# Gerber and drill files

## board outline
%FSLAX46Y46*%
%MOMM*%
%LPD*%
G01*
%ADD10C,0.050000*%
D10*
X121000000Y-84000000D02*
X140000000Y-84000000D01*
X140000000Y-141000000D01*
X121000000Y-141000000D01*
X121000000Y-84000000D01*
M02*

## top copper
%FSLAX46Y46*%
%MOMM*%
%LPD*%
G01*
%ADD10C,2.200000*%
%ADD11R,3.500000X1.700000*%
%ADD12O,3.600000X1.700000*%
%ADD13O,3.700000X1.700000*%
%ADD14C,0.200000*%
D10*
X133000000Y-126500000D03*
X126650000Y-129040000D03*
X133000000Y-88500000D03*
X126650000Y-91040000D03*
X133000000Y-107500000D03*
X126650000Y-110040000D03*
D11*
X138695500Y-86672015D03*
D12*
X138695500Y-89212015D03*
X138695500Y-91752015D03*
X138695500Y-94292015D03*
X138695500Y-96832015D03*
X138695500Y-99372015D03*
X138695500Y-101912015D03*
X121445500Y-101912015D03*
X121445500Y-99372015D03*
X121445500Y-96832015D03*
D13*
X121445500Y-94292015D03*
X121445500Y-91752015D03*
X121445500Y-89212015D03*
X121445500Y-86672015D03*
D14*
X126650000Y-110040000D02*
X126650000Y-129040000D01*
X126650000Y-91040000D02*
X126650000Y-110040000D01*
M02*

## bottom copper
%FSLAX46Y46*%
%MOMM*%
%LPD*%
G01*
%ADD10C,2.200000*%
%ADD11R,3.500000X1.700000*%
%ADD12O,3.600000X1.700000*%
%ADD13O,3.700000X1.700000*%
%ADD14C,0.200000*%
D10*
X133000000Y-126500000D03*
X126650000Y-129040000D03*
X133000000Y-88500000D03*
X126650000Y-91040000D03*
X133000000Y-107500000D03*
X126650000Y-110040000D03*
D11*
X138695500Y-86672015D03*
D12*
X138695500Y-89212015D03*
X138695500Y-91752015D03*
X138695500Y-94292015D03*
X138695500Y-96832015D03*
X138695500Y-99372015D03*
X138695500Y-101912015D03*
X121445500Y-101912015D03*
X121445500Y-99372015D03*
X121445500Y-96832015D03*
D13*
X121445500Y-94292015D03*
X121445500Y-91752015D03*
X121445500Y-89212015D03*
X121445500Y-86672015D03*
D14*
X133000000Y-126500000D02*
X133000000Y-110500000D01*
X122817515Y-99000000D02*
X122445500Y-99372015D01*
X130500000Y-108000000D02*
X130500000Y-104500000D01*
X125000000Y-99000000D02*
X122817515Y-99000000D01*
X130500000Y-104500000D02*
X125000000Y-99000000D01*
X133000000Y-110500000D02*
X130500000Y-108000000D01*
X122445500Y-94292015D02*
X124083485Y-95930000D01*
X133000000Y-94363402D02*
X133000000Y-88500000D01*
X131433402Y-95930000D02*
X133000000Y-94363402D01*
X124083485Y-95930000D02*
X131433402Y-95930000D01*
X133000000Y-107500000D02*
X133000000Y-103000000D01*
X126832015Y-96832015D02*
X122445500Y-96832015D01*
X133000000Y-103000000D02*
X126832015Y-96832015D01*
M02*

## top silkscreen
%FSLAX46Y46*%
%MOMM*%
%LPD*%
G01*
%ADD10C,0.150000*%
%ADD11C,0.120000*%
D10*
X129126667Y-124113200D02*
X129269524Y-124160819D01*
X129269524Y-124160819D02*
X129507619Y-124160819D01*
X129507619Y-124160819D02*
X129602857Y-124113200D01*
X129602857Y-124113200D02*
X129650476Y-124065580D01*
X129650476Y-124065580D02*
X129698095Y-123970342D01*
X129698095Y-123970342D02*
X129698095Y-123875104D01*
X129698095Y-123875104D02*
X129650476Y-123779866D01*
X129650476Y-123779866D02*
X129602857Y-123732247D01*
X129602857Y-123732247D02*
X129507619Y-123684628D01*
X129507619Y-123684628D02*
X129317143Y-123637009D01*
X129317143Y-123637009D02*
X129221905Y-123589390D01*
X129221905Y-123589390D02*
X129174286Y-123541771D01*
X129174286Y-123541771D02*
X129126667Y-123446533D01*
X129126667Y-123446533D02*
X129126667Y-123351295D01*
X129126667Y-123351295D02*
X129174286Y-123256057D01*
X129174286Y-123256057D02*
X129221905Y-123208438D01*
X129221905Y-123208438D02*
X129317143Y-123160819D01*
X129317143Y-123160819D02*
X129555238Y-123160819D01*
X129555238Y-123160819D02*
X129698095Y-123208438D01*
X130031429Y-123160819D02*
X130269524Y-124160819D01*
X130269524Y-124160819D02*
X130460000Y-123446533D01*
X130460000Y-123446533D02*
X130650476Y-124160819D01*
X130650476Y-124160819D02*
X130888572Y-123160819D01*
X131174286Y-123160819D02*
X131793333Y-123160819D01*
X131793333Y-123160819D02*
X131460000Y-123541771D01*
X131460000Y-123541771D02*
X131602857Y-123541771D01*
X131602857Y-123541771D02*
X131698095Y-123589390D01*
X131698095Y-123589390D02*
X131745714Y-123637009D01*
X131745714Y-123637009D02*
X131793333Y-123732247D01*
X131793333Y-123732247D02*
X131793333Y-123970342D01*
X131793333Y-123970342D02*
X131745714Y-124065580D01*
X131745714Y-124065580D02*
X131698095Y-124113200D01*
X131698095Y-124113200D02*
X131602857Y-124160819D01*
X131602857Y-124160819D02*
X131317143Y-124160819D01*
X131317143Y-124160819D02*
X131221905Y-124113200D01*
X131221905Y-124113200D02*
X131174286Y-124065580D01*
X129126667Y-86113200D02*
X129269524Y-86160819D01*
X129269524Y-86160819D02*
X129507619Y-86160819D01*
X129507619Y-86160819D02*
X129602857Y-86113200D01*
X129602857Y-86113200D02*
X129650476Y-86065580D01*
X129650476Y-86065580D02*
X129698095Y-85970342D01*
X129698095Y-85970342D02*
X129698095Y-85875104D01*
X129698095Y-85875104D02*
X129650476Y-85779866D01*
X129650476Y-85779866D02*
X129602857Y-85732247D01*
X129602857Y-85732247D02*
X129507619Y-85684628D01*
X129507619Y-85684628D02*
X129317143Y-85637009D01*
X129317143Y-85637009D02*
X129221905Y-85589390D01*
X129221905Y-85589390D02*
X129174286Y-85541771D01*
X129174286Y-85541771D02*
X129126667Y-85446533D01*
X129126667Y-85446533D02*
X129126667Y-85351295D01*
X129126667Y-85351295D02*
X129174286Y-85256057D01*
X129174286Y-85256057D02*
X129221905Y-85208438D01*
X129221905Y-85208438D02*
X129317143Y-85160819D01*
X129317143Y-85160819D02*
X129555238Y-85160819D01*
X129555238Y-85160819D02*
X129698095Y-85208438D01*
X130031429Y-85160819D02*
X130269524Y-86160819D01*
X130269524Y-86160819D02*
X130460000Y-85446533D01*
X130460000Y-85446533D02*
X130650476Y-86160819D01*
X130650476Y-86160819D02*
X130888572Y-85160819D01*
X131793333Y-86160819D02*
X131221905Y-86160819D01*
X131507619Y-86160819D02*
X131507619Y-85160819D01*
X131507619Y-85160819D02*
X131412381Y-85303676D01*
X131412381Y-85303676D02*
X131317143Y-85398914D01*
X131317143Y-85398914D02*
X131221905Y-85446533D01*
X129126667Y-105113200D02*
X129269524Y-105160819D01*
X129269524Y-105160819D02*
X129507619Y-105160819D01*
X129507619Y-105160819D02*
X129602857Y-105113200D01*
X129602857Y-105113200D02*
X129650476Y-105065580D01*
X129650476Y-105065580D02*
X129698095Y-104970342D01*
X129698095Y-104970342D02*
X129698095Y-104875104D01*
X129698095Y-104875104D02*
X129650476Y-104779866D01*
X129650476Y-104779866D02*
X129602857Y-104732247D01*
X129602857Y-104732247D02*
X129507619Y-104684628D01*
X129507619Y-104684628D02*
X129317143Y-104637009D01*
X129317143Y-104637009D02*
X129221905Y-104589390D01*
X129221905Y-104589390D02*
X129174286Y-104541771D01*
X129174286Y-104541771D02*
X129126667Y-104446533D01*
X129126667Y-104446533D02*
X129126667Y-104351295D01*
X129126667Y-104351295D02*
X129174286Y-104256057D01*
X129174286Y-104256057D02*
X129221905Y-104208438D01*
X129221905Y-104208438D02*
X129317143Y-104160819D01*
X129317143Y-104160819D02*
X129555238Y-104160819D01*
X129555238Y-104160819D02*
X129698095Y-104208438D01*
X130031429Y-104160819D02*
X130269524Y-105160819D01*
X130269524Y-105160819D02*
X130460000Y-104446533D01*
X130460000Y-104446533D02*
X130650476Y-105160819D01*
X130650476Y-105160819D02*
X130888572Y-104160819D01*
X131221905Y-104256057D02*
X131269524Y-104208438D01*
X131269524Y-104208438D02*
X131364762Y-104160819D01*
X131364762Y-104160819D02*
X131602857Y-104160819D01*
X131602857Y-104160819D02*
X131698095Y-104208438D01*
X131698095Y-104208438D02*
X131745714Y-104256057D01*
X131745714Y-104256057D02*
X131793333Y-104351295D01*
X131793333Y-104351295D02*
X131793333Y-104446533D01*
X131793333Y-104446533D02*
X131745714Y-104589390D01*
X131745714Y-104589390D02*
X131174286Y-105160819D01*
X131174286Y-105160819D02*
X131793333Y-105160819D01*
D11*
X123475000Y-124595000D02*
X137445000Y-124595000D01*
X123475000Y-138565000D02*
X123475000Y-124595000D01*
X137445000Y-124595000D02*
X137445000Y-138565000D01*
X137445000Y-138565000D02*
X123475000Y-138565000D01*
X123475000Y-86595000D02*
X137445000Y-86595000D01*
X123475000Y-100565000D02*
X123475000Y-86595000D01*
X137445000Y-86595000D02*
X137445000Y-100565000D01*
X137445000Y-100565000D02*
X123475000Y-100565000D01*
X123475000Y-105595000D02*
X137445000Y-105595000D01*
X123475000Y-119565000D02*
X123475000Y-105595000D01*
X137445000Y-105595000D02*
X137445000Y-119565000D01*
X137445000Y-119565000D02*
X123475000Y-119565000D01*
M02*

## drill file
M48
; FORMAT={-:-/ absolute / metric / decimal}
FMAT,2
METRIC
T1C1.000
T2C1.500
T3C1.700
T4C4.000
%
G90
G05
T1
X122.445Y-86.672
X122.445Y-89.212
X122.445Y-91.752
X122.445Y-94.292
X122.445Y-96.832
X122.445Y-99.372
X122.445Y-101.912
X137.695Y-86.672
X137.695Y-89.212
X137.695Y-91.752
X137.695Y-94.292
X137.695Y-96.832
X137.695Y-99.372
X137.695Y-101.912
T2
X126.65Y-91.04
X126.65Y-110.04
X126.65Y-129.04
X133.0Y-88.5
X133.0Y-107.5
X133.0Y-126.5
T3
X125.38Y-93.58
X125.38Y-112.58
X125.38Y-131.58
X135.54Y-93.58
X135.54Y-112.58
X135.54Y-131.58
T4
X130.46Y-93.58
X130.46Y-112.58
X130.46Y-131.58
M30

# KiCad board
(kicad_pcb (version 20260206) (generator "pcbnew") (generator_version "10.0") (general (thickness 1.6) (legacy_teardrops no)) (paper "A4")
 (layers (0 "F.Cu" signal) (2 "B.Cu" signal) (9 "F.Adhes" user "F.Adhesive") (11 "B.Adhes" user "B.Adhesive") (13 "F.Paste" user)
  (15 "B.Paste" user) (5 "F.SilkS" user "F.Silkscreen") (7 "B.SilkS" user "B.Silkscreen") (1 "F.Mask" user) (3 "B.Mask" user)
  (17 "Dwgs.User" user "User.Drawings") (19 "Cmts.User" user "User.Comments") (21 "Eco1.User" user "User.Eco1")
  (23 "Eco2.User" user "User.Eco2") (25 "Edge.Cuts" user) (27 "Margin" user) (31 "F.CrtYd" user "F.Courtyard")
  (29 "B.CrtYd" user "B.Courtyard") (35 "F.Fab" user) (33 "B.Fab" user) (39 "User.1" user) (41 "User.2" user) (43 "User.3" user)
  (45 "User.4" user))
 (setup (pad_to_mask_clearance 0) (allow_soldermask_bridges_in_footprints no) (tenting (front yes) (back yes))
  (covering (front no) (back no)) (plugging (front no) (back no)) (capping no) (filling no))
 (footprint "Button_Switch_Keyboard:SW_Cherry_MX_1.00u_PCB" (layer "F.Cu") (at 133 126.5)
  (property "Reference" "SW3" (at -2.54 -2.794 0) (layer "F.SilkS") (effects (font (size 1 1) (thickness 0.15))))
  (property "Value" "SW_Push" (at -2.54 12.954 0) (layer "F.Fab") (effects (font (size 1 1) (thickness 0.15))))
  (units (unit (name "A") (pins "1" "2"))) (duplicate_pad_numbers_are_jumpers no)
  (fp_line (start -9.525 -1.905) (end 4.445 -1.905) (stroke (width 0.12) (type solid)) (layer "F.SilkS"))
  (fp_line (start -9.525 12.065) (end -9.525 -1.905) (stroke (width 0.12) (type solid)) (layer "F.SilkS"))
  (fp_line (start 4.445 -1.905) (end 4.445 12.065) (stroke (width 0.12) (type solid)) (layer "F.SilkS"))
  (fp_line (start 4.445 12.065) (end -9.525 12.065) (stroke (width 0.12) (type solid)) (layer "F.SilkS"))
  (pad "" np_thru_hole circle (at -7.62 5.08) (size 1.7 1.7) (drill 1.7) (layers "*.Cu" "*.Mask"))
  (pad "" np_thru_hole circle (at -2.54 5.08) (size 4 4) (drill 4) (layers "*.Cu" "*.Mask"))
  (pad "" np_thru_hole circle (at 2.54 5.08) (size 1.7 1.7) (drill 1.7) (layers "*.Cu" "*.Mask"))
  (pad "1" thru_hole circle (at 0 0) (size 2.2 2.2) (drill 1.5) (layers "*.Cu" "*.Mask") (remove_unused_layers no)
   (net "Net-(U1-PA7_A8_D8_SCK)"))
  (pad "2" thru_hole circle (at -6.35 2.54) (size 2.2 2.2) (drill 1.5) (layers "*.Cu" "*.Mask") (remove_unused_layers no) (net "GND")))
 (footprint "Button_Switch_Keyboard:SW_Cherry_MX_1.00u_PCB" (layer "F.Cu") (at 133 88.5)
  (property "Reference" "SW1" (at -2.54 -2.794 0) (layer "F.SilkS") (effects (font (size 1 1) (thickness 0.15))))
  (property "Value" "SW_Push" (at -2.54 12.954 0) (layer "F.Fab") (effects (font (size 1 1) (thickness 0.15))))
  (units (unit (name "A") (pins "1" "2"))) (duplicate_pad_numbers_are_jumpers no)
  (fp_line (start -9.525 -1.905) (end 4.445 -1.905) (stroke (width 0.12) (type solid)) (layer "F.SilkS"))
  (fp_line (start -9.525 12.065) (end -9.525 -1.905) (stroke (width 0.12) (type solid)) (layer "F.SilkS"))
  (fp_line (start 4.445 -1.905) (end 4.445 12.065) (stroke (width 0.12) (type solid)) (layer "F.SilkS"))
  (fp_line (start 4.445 12.065) (end -9.525 12.065) (stroke (width 0.12) (type solid)) (layer "F.SilkS"))
  (pad "" np_thru_hole circle (at -7.62 5.08) (size 1.7 1.7) (drill 1.7) (layers "*.Cu" "*.Mask"))
  (pad "" np_thru_hole circle (at -2.54 5.08) (size 4 4) (drill 4) (layers "*.Cu" "*.Mask"))
  (pad "" np_thru_hole circle (at 2.54 5.08) (size 1.7 1.7) (drill 1.7) (layers "*.Cu" "*.Mask"))
  (pad "1" thru_hole circle (at 0 0) (size 2.2 2.2) (drill 1.5) (layers "*.Cu" "*.Mask") (remove_unused_layers no)
   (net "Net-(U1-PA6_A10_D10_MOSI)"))
  (pad "2" thru_hole circle (at -6.35 2.54) (size 2.2 2.2) (drill 1.5) (layers "*.Cu" "*.Mask") (remove_unused_layers no) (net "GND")))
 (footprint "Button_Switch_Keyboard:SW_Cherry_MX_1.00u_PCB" (layer "F.Cu") (at 133 107.5)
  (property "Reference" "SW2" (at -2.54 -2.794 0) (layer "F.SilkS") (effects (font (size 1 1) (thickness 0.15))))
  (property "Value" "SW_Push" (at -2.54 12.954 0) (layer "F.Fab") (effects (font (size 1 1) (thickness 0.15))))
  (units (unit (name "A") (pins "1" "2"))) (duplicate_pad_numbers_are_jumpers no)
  (fp_line (start -9.525 -1.905) (end 4.445 -1.905) (stroke (width 0.12) (type solid)) (layer "F.SilkS"))
  (fp_line (start -9.525 12.065) (end -9.525 -1.905) (stroke (width 0.12) (type solid)) (layer "F.SilkS"))
  (fp_line (start 4.445 -1.905) (end 4.445 12.065) (stroke (width 0.12) (type solid)) (layer "F.SilkS"))
  (fp_line (start 4.445 12.065) (end -9.525 12.065) (stroke (width 0.12) (type solid)) (layer "F.SilkS"))
  (pad "" np_thru_hole circle (at -7.62 5.08) (size 1.7 1.7) (drill 1.7) (layers "*.Cu" "*.Mask"))
  (pad "" np_thru_hole circle (at -2.54 5.08) (size 4 4) (drill 4) (layers "*.Cu" "*.Mask"))
  (pad "" np_thru_hole circle (at 2.54 5.08) (size 1.7 1.7) (drill 1.7) (layers "*.Cu" "*.Mask"))
  (pad "1" thru_hole circle (at 0 0) (size 2.2 2.2) (drill 1.5) (layers "*.Cu" "*.Mask") (remove_unused_layers no)
   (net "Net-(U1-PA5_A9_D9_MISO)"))
  (pad "2" thru_hole circle (at -6.35 2.54) (size 2.2 2.2) (drill 1.5) (layers "*.Cu" "*.Mask") (remove_unused_layers no) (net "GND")))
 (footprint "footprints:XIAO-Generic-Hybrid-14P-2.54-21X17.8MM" (layer "B.Cu") (at 130.0705 94.292015 180)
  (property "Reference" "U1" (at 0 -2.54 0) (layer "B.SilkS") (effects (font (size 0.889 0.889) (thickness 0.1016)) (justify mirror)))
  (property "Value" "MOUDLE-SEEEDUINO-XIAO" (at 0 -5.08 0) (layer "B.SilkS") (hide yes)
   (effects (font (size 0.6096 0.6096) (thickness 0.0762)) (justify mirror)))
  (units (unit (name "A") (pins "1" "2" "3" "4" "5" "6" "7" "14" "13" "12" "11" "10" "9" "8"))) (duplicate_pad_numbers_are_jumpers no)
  (pad "1" thru_hole rect (at -7.625 7.62 180) (size 3.5 1.7) (drill 1 (offset -1 0)) (layers "*.Cu" "*.Mask") (remove_unused_layers no)
   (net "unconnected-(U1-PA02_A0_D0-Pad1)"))
  (pad "2" thru_hole oval (at -7.625 5.08 180) (size 3.6 1.7) (drill 1 (offset -1 0)) (layers "*.Cu" "*.Mask") (remove_unused_layers no)
   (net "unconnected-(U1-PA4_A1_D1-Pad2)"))
  (pad "3" thru_hole oval (at -7.625 2.54 180) (size 3.6 1.7) (drill 1 (offset -1 0)) (layers "*.Cu" "*.Mask") (remove_unused_layers no)
   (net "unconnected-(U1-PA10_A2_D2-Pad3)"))
  (pad "4" thru_hole oval (at -7.625 0 180) (size 3.6 1.7) (drill 1 (offset -1 0)) (layers "*.Cu" "*.Mask") (remove_unused_layers no)
   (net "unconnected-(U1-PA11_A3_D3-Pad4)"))
  (pad "5" thru_hole oval (at -7.625 -2.54 180) (size 3.6 1.7) (drill 1 (offset -1 0)) (layers "*.Cu" "*.Mask") (remove_unused_layers no)
   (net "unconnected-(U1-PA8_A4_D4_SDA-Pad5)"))
  (pad "6" thru_hole oval (at -7.625 -5.08) (size 3.6 1.7) (drill 1 (offset 1 0)) (layers "*.Cu" "*.Mask") (remove_unused_layers no)
   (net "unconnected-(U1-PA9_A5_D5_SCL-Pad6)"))
  (pad "7" thru_hole oval (at -7.625 -7.62 180) (size 3.6 1.7) (drill 1 (offset -1 0)) (layers "*.Cu" "*.Mask") (remove_unused_layers no)
   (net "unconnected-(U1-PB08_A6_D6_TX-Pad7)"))
  (pad "8" thru_hole oval (at 7.625 -7.62 180) (size 3.6 1.7) (drill 1 (offset 1 0)) (layers "*.Cu" "*.Mask") (remove_unused_layers no)
   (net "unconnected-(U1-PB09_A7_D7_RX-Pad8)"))
  (pad "9" thru_hole oval (at 7.625 -5.08 180) (size 3.6 1.7) (drill 1 (offset 1 0)) (layers "*.Cu" "*.Mask") (remove_unused_layers no)
   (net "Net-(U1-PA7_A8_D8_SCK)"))
  (pad "10" thru_hole oval (at 7.625 -2.54 180) (size 3.6 1.7) (drill 1 (offset 1 0)) (layers "*.Cu" "*.Mask") (remove_unused_layers no)
   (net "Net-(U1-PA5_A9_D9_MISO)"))
  (pad "11" thru_hole oval (at 7.625 0 180) (size 3.7 1.7) (drill 1 (offset 1 0)) (layers "*.Cu" "*.Mask") (remove_unused_layers no)
   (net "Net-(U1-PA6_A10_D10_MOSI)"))
  (pad "12" thru_hole oval (at 7.625 2.54 180) (size 3.7 1.7) (drill 1 (offset 1 0)) (layers "*.Cu" "*.Mask") (remove_unused_layers no)
   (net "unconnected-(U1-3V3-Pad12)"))
  (pad "13" thru_hole oval (at 7.625 5.08 180) (size 3.7 1.7) (drill 1 (offset 1 0)) (layers "*.Cu" "*.Mask") (remove_unused_layers no)
   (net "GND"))
  (pad "14" thru_hole oval (at 7.625 7.62 180) (size 3.7 1.7) (drill 1 (offset 1 0)) (layers "*.Cu" "*.Mask") (remove_unused_layers no)
   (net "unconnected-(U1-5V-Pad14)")))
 (gr_rect (start 121 84) (end 140 141) (stroke (width 0.05) (type default)) (fill no) (layer "Edge.Cuts"))
 (segment (start 133 126.5) (end 133 110.5) (width 0.2) (layer "B.Cu") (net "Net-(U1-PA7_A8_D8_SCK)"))
 (segment (start 122.817515 99) (end 122.4455 99.372015) (width 0.2) (layer "B.Cu") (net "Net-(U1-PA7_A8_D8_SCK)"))
 (segment (start 130.5 108) (end 130.5 104.5) (width 0.2) (layer "B.Cu") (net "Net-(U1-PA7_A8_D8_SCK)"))
 (segment (start 125 99) (end 122.817515 99) (width 0.2) (layer "B.Cu") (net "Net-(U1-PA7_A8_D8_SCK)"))
 (segment (start 130.5 104.5) (end 125 99) (width 0.2) (layer "B.Cu") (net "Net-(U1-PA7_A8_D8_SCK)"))
 (segment (start 133 110.5) (end 130.5 108) (width 0.2) (layer "B.Cu") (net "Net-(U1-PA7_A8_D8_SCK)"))
 (segment (start 126.65 110.04) (end 126.65 129.04) (width 0.2) (layer "F.Cu") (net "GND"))
 (segment (start 126.65 91.04) (end 126.65 110.04) (width 0.2) (layer "F.Cu") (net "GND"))
 (segment (start 122.4455 94.292015) (end 124.083485 95.93) (width 0.2) (layer "B.Cu") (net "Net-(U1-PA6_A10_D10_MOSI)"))
 (segment (start 133 94.363402) (end 133 88.5) (width 0.2) (layer "B.Cu") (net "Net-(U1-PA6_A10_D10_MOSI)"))
 (segment (start 131.433402 95.93) (end 133 94.363402) (width 0.2) (layer "B.Cu") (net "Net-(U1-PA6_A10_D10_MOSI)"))
 (segment (start 124.083485 95.93) (end 131.433402 95.93) (width 0.2) (layer "B.Cu") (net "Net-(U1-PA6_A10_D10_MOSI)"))
 (segment (start 133 107.5) (end 133 103) (width 0.2) (layer "B.Cu") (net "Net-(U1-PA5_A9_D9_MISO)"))
 (segment (start 126.832015 96.832015) (end 122.4455 96.832015) (width 0.2) (layer "B.Cu") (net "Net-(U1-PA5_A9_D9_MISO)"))
 (segment (start 133 103) (end 126.832015 96.832015) (width 0.2) (layer "B.Cu") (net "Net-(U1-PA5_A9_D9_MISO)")))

